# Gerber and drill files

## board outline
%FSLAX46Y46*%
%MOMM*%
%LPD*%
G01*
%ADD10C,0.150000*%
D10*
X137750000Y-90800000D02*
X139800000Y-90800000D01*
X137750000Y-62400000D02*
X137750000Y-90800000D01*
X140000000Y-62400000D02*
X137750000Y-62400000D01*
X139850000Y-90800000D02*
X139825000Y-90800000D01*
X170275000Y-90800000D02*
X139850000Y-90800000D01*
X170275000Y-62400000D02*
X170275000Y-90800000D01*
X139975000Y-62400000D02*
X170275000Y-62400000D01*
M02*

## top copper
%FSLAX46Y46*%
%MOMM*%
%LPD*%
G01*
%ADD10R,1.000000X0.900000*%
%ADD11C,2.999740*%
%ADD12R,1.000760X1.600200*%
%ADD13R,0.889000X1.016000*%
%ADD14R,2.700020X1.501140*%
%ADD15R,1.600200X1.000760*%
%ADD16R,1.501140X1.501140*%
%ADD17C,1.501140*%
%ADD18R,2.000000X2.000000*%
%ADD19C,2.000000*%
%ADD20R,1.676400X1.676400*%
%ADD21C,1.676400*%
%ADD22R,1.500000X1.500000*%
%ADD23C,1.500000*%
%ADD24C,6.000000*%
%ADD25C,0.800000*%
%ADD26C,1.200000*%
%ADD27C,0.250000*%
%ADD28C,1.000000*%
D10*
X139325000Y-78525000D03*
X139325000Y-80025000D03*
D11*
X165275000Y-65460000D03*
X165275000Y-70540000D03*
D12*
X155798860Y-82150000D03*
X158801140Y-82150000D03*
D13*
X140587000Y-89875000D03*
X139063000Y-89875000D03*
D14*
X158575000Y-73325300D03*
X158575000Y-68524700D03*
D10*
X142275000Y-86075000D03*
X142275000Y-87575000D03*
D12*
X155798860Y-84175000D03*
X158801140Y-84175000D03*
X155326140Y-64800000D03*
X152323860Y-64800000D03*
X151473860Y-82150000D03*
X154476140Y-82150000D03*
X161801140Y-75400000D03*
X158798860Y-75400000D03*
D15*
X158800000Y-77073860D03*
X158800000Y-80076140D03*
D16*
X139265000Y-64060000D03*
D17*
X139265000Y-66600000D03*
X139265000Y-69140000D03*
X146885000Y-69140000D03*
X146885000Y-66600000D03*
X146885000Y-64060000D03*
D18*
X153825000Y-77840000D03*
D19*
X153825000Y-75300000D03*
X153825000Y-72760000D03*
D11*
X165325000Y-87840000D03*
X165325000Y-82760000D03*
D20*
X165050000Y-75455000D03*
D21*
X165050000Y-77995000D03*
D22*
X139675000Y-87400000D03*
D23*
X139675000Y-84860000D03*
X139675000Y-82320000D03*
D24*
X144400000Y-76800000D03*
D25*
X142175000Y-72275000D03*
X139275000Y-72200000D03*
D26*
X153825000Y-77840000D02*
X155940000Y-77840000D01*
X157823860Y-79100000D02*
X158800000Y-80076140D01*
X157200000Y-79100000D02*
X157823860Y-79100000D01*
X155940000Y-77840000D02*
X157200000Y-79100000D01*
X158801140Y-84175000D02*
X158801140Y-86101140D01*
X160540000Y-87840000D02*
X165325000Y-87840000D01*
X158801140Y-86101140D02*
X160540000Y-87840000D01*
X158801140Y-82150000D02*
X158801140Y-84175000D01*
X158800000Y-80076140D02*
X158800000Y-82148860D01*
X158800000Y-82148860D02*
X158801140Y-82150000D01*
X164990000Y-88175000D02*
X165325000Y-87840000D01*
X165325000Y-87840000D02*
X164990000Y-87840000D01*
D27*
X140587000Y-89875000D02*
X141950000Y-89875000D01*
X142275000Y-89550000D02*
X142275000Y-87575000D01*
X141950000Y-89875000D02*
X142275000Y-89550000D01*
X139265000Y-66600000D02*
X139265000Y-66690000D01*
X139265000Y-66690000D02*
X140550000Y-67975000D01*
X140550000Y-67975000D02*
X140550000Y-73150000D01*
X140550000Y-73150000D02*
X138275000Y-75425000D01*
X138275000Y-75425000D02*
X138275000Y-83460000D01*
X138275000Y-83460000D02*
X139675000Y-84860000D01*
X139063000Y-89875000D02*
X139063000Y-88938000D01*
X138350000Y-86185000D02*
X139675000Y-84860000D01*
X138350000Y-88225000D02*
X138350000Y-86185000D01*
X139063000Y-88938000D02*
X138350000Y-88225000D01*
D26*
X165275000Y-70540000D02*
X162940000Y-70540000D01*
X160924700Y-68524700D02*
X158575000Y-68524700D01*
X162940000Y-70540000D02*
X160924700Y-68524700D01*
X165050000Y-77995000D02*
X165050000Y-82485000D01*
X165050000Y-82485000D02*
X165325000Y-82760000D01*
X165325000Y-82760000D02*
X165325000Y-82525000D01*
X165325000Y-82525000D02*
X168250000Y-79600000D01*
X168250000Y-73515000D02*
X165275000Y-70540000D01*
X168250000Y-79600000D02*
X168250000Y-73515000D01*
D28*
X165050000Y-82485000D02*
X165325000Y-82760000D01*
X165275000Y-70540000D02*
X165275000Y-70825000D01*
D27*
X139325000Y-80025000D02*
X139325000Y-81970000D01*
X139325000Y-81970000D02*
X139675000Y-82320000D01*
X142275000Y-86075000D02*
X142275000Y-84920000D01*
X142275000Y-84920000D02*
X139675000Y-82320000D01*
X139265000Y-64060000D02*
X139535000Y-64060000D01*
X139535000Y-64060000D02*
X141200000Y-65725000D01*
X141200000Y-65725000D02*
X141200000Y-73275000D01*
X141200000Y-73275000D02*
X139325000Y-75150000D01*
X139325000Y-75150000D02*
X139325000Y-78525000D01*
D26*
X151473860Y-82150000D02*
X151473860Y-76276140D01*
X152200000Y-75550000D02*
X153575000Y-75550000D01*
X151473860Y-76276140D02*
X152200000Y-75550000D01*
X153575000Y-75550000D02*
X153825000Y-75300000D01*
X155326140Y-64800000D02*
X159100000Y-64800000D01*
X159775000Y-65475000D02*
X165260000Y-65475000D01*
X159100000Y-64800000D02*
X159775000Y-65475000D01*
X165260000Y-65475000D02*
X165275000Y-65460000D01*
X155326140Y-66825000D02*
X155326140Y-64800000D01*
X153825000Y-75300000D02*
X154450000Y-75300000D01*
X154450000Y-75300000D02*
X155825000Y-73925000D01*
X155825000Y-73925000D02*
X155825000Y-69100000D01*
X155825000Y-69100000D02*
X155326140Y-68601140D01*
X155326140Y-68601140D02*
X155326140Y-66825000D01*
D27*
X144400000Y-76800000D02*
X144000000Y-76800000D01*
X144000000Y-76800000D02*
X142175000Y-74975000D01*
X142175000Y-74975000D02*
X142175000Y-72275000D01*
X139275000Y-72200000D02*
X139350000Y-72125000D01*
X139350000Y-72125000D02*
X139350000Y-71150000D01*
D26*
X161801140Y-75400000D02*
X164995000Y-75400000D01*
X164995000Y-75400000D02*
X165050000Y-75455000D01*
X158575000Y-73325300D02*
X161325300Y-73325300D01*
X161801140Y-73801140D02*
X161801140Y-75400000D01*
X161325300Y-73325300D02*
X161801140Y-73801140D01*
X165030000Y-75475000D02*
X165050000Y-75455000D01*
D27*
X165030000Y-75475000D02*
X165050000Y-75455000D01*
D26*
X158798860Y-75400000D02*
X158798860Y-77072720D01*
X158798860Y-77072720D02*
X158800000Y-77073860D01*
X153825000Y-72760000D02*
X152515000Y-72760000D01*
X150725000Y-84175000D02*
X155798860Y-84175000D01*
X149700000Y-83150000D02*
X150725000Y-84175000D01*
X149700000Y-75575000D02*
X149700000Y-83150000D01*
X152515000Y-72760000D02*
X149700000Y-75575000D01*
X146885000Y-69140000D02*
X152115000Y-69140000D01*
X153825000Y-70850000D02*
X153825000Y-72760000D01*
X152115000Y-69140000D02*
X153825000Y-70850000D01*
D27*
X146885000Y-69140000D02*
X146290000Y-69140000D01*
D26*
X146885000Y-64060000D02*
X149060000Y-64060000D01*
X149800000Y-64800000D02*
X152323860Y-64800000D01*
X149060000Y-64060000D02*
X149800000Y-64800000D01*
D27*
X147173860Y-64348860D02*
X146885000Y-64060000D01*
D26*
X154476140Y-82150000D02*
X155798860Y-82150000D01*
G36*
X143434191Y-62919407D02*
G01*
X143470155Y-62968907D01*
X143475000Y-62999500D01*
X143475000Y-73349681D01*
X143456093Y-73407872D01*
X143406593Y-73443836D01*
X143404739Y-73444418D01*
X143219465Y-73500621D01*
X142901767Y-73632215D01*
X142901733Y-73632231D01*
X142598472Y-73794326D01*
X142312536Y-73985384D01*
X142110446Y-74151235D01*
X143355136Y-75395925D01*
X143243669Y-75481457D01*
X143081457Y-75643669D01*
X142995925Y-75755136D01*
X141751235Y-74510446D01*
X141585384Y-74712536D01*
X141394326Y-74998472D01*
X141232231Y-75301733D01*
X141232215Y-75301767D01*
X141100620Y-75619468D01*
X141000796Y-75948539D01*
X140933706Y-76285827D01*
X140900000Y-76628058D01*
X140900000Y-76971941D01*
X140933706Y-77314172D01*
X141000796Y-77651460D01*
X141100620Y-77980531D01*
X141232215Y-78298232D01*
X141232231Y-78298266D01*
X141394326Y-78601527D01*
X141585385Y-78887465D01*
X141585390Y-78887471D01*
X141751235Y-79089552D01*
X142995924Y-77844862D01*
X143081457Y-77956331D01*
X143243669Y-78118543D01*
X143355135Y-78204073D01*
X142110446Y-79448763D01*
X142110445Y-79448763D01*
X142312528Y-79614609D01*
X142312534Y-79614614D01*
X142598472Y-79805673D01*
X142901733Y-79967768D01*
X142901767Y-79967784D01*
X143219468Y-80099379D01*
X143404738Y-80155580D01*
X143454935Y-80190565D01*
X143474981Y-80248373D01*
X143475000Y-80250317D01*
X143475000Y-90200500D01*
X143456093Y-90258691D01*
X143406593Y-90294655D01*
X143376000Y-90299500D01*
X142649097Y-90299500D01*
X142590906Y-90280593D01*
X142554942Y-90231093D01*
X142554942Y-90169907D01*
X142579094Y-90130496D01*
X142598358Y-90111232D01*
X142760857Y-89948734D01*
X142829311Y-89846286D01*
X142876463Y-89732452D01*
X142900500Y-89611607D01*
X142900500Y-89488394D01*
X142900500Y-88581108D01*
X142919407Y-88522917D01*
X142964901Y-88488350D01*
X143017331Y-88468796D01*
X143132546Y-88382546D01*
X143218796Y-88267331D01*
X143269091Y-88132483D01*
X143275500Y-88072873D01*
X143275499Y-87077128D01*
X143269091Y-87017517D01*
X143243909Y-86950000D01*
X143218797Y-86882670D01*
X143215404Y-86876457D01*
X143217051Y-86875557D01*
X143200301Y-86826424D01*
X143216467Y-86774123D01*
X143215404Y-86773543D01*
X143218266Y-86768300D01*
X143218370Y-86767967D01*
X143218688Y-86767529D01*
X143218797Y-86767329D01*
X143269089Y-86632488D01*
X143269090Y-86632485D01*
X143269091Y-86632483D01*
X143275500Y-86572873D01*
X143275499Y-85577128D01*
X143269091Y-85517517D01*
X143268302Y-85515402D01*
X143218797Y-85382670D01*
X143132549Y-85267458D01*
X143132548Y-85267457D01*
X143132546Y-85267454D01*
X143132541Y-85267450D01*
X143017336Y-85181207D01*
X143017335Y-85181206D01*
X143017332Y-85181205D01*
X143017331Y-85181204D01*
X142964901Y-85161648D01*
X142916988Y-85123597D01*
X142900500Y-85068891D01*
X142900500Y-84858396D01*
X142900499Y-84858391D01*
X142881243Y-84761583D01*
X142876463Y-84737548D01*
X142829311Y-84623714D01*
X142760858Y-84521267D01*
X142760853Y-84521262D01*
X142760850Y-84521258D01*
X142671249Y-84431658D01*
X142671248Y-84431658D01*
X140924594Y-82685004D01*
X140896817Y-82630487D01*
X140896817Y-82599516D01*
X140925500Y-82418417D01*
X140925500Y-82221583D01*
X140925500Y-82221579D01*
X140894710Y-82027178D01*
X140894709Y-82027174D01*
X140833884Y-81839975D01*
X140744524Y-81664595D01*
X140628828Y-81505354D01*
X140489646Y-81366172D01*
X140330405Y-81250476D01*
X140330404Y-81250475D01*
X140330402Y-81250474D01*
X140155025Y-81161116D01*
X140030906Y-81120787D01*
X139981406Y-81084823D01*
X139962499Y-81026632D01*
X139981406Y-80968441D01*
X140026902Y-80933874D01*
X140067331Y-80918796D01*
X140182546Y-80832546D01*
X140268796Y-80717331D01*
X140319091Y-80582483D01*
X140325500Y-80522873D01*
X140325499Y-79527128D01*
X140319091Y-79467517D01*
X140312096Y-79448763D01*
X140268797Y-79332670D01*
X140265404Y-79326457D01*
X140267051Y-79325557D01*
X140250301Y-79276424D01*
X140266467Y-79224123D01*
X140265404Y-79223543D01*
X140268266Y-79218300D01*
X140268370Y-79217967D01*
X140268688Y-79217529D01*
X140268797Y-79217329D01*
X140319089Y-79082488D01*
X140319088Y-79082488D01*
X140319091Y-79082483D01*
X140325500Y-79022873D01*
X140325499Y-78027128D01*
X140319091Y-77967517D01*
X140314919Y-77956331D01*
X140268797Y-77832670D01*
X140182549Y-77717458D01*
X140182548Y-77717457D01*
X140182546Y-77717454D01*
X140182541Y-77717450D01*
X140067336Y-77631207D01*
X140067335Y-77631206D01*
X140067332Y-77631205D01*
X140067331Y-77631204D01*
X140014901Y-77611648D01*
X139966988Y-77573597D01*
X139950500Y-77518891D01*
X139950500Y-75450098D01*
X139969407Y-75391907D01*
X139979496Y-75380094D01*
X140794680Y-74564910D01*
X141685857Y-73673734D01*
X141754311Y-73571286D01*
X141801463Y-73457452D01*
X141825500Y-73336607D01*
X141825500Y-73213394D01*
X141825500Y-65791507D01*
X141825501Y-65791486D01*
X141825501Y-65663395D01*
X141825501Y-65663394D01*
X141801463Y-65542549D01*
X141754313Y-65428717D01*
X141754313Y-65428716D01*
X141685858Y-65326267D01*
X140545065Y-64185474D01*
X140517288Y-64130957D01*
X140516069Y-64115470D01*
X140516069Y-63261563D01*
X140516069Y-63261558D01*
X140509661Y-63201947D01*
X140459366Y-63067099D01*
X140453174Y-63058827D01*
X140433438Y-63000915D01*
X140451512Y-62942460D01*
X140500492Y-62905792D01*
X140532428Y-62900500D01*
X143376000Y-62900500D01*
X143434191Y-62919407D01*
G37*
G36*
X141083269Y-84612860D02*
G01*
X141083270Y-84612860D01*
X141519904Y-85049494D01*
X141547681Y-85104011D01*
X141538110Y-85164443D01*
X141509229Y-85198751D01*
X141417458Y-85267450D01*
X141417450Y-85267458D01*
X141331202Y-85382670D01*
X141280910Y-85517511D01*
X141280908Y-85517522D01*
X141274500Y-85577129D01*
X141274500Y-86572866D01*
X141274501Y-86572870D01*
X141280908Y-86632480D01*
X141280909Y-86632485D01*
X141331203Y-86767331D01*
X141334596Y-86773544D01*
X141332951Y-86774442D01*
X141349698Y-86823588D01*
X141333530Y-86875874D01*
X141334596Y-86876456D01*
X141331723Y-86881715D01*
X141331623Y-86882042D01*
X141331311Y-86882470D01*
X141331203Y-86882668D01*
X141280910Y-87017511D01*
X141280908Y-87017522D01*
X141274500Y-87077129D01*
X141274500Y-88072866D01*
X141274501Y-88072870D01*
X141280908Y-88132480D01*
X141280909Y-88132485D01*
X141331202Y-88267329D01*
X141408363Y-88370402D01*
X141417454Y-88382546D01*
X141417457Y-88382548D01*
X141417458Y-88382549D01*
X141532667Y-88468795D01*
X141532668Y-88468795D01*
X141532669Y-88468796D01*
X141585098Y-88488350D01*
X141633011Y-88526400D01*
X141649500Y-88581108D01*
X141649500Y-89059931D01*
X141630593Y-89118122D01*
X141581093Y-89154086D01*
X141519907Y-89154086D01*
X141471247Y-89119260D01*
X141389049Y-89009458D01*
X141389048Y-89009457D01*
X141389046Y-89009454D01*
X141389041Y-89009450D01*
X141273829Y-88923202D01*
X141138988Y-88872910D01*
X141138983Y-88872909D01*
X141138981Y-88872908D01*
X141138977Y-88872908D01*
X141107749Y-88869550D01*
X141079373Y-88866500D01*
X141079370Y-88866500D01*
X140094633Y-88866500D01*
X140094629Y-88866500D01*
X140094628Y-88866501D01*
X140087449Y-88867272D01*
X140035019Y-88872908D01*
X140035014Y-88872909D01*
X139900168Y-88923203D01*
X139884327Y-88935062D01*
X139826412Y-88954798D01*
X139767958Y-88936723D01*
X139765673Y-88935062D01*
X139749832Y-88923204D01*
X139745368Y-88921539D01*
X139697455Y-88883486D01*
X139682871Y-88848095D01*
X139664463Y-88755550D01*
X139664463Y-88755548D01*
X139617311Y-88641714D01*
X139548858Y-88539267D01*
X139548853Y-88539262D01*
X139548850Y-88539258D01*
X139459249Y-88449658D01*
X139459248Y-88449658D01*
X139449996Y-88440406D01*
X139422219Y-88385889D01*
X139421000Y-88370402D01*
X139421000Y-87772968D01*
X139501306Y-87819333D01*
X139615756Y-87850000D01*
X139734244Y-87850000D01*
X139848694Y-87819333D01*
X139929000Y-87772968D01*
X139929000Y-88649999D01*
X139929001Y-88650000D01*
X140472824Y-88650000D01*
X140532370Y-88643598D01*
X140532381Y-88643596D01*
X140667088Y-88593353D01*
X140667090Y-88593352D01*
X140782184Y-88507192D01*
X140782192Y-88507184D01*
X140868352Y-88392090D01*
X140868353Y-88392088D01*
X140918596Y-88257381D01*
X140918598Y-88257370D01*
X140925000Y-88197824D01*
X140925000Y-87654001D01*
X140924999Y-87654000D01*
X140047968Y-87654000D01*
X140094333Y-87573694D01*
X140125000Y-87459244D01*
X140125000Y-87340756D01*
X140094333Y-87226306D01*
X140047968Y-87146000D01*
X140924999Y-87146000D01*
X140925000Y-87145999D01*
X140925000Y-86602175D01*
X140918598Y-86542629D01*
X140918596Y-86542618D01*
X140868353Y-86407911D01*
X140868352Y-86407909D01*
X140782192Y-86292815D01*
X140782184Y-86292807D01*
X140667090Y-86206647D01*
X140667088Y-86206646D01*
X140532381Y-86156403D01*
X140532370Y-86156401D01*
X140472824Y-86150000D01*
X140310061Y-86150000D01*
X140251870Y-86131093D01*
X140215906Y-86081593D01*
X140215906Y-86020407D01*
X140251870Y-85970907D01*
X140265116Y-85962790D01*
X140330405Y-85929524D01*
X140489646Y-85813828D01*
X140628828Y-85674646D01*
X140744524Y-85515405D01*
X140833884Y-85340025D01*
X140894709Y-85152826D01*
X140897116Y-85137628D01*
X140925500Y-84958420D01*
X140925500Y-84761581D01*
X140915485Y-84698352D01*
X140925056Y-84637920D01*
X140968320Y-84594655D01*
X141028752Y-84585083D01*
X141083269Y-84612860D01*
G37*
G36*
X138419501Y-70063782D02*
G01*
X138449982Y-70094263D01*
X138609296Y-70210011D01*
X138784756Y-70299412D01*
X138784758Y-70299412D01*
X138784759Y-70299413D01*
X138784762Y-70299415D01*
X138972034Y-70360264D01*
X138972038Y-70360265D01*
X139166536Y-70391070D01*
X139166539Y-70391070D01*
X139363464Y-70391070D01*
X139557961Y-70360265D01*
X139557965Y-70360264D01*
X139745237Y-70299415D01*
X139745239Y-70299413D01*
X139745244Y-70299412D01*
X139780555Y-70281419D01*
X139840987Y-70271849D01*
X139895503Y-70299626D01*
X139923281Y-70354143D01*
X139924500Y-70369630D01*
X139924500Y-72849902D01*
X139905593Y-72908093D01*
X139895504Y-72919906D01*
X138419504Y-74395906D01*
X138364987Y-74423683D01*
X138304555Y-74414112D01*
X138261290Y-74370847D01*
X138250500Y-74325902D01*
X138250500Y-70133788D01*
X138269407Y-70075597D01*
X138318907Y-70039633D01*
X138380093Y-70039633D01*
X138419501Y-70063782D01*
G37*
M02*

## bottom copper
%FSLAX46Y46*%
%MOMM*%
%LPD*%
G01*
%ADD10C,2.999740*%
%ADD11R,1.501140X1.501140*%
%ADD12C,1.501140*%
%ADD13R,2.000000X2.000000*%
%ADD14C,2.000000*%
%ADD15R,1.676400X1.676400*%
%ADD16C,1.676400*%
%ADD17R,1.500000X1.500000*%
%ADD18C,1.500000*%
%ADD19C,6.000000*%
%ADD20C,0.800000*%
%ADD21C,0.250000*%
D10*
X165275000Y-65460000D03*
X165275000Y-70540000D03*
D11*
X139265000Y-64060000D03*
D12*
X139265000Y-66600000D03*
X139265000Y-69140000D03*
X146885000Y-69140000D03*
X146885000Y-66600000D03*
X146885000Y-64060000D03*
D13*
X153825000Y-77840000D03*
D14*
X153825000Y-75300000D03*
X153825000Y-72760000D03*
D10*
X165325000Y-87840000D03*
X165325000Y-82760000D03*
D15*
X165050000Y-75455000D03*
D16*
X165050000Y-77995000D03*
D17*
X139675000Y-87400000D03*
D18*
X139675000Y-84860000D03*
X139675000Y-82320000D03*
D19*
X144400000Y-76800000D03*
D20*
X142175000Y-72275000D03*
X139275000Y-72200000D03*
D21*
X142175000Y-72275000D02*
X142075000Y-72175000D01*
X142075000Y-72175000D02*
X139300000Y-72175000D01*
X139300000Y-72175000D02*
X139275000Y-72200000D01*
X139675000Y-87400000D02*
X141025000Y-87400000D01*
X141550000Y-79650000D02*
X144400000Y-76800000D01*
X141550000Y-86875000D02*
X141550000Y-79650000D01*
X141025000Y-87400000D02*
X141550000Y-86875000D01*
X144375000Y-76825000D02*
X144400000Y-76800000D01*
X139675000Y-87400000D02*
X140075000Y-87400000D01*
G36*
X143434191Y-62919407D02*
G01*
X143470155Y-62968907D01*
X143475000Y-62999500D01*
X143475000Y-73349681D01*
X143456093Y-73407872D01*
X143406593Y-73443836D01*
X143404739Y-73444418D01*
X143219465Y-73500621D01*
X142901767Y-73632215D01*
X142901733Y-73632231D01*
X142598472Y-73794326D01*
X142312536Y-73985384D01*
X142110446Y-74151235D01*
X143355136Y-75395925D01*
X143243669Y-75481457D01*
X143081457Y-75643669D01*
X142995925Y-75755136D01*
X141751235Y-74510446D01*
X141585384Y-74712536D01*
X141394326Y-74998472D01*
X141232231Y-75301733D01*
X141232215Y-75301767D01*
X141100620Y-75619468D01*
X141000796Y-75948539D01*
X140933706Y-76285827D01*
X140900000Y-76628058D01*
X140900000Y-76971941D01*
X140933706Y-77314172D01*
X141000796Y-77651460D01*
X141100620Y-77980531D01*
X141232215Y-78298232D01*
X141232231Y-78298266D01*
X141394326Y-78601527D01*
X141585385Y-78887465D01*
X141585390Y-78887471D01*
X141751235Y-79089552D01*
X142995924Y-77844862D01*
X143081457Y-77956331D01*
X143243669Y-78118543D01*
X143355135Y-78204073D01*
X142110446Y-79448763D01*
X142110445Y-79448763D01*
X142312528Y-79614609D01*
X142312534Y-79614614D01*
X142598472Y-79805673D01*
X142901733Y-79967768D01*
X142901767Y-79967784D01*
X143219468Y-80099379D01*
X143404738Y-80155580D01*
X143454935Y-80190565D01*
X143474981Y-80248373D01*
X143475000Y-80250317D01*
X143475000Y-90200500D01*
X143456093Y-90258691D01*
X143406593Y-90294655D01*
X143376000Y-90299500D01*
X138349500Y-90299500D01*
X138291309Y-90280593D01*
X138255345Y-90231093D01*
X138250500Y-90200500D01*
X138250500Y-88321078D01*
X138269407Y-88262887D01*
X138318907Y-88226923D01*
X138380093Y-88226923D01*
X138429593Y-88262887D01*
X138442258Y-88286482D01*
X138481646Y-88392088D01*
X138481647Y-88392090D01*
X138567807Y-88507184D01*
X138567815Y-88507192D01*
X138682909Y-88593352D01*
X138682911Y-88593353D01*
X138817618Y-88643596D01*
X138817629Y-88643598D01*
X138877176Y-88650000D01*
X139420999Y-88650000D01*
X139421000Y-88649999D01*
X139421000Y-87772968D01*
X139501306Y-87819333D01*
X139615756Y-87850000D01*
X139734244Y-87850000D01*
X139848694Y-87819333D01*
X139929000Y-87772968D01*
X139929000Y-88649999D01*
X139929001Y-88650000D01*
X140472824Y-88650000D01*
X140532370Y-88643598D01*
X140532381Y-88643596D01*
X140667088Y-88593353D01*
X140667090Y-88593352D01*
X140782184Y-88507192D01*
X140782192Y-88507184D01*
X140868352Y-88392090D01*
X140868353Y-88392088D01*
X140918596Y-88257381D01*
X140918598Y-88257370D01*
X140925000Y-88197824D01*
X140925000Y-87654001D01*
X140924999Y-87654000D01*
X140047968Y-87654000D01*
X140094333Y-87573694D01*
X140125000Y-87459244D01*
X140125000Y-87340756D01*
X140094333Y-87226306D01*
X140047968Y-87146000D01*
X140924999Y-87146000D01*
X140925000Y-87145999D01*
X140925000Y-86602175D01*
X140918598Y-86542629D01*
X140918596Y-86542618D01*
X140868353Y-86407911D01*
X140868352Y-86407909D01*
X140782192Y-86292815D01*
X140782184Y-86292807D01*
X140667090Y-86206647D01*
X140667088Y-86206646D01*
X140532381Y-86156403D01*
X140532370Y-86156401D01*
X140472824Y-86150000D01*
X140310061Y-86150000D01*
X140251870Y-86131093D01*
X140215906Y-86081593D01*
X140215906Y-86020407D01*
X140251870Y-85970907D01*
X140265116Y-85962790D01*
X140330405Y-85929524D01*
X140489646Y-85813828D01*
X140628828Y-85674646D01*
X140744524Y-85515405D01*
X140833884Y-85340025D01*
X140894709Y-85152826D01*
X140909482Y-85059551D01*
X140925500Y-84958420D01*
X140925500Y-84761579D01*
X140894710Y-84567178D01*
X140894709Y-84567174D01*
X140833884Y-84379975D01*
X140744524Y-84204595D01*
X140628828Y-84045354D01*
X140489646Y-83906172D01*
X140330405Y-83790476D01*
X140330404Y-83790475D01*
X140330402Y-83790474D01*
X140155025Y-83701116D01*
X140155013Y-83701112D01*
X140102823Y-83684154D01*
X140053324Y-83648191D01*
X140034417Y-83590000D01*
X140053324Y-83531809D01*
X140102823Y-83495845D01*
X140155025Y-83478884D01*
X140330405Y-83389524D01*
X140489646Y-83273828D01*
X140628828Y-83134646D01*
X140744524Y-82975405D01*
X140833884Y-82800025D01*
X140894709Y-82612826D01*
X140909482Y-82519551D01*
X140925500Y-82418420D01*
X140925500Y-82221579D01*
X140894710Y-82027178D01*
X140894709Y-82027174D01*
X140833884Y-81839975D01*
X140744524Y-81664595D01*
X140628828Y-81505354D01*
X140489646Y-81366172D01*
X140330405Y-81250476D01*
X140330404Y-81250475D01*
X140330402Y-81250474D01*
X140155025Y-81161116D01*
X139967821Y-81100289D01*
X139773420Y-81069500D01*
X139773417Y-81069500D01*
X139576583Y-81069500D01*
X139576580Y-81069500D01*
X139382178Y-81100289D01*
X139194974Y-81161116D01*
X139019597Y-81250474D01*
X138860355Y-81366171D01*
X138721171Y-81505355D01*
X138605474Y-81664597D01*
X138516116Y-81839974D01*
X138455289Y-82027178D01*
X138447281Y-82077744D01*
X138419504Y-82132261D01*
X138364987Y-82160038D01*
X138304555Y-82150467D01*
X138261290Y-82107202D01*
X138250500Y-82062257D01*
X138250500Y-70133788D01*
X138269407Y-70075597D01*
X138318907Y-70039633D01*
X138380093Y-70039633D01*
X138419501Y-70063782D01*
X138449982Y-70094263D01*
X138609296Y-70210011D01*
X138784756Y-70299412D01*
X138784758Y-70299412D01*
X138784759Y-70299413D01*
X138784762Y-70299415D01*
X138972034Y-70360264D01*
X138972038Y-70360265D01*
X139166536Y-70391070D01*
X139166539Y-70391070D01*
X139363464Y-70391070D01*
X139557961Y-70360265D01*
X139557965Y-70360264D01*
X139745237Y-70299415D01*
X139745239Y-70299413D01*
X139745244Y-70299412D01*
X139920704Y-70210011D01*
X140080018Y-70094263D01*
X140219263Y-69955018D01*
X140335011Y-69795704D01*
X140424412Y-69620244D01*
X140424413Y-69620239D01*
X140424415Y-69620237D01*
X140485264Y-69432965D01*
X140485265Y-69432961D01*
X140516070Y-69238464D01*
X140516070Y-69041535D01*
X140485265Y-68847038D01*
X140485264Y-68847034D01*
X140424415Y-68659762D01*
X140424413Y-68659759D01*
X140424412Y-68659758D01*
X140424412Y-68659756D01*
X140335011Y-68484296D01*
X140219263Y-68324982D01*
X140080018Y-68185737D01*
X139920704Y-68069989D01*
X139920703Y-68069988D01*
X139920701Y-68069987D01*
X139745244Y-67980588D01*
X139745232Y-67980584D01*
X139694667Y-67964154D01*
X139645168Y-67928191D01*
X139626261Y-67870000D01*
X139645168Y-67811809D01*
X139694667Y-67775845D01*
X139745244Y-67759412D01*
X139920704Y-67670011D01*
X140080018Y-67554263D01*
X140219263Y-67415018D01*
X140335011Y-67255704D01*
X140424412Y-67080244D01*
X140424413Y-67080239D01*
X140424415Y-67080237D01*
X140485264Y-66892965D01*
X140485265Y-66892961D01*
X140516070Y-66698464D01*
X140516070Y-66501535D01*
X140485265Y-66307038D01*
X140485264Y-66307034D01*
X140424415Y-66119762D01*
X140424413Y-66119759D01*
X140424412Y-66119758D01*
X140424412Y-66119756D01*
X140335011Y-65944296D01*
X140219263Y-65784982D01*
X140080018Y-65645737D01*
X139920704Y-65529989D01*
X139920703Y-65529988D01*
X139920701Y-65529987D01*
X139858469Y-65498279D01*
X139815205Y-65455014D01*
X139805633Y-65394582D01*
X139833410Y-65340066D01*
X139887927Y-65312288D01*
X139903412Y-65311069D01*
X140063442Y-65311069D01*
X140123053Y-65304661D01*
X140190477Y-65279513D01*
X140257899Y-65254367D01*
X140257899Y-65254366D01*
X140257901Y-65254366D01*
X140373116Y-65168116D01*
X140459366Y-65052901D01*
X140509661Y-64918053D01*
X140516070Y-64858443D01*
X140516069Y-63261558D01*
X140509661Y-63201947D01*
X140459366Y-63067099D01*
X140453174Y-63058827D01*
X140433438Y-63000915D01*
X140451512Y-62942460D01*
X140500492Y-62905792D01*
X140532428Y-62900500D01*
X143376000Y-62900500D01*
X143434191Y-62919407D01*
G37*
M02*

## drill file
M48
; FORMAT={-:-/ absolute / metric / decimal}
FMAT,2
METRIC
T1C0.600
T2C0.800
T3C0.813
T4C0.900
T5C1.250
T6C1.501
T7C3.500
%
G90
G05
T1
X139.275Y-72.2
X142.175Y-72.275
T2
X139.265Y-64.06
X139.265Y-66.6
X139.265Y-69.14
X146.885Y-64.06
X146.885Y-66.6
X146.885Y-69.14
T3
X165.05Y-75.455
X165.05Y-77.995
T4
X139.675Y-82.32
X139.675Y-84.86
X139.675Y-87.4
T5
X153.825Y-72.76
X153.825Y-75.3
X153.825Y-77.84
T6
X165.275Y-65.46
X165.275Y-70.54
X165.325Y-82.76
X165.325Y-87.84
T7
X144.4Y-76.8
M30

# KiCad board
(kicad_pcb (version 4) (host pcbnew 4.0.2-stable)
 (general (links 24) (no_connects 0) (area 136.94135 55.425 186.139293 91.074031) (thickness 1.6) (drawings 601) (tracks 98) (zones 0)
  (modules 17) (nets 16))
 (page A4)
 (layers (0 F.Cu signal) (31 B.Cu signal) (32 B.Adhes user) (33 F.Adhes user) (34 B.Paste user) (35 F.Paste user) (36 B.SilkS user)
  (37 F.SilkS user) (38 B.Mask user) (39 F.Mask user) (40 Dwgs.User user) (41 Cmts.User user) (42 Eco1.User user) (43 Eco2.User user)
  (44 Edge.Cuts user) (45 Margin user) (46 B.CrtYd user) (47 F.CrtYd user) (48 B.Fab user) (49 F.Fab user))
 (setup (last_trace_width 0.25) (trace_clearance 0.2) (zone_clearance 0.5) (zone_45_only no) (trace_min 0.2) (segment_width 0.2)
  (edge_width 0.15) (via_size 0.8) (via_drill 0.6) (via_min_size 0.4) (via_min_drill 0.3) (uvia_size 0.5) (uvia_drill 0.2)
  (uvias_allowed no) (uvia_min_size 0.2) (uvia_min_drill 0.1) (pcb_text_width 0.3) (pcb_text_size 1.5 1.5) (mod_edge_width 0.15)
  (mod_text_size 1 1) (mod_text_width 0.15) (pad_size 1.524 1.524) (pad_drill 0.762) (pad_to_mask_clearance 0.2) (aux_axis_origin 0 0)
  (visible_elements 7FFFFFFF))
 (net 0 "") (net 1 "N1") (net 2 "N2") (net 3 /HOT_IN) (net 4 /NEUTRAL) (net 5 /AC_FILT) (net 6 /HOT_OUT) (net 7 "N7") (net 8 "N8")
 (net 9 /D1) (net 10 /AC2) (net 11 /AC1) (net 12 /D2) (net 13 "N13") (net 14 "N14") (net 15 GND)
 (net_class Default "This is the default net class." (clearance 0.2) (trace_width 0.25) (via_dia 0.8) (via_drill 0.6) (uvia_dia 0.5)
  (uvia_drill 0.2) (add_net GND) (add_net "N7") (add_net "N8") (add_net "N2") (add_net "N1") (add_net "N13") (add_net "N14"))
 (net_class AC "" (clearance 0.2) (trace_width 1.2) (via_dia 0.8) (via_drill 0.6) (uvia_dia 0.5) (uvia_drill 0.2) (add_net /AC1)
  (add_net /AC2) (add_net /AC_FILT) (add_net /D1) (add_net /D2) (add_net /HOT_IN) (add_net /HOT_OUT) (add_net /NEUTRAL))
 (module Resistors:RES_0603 (layer F.Cu) (at 139.325 79.275 270)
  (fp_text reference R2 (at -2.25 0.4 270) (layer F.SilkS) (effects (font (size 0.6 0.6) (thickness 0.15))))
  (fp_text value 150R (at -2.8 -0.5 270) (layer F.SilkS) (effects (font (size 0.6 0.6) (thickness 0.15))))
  (pad 1 smd rect (at -0.75 0 270) (size 0.9 1) (layers F.Cu F.Paste F.Mask) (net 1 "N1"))
  (pad 2 smd rect (at 0.75 0 270) (size 0.9 1) (layers F.Cu F.Paste F.Mask) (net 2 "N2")))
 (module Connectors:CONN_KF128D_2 (layer F.Cu) (at 165.275 68 270)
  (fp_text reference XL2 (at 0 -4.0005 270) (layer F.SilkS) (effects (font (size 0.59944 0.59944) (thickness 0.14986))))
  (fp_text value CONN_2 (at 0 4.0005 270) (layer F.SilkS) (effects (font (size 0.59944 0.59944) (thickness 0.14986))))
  (pad 1 thru_hole circle (at -2.54 0 270) (size 2.99974 2.99974) (drill 1.50114) (layers *.Cu *.Mask F.SilkS) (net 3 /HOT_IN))
  (pad 2 thru_hole circle (at 2.54 0 270) (size 2.99974 2.99974) (drill 1.50114) (layers *.Cu *.Mask F.SilkS) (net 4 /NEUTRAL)))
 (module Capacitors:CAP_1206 (layer F.Cu) (at 157.3 82.15)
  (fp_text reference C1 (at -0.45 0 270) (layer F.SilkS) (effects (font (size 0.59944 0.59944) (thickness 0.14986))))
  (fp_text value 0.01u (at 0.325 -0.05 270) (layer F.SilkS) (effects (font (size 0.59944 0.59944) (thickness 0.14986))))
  (pad 1 smd rect (at -1.50114 0) (size 1.00076 1.6002) (layers F.Cu F.Paste F.Mask) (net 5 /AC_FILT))
  (pad 2 smd rect (at 1.50114 0) (size 1.00076 1.6002) (layers F.Cu F.Paste F.Mask) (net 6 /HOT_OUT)))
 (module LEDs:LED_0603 (layer F.Cu) (at 139.825 89.875 180)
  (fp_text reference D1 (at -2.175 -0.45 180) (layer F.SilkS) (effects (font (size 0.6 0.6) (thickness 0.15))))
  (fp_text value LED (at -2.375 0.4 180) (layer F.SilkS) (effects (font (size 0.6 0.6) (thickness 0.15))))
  (pad A smd rect (at -0.762 0 180) (size 0.889 1.016) (layers F.Cu F.Paste F.Mask) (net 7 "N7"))
  (pad C smd rect (at 0.762 0 180) (size 0.889 1.016) (layers F.Cu F.Paste F.Mask) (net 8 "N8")))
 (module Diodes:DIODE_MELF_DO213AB (layer F.Cu) (at 158.575 70.925 90)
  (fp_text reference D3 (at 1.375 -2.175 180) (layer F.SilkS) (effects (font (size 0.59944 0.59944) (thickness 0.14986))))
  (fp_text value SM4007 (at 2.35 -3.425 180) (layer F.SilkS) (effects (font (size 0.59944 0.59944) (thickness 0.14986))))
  (pad C smd rect (at -2.4003 0 90) (size 1.50114 2.70002) (layers F.Cu F.Paste F.Mask) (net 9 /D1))
  (pad A smd rect (at 2.4003 0 90) (size 1.50114 2.70002) (layers F.Cu F.Paste F.Mask) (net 4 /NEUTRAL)))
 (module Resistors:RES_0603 (layer F.Cu) (at 142.275 86.825 270)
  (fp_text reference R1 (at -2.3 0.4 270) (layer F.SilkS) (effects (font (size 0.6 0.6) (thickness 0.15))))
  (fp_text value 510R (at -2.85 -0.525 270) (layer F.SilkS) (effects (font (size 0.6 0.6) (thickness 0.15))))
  (pad 1 smd rect (at -0.75 0 270) (size 0.9 1) (layers F.Cu F.Paste F.Mask) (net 2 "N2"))
  (pad 2 smd rect (at 0.75 0 270) (size 0.9 1) (layers F.Cu F.Paste F.Mask) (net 7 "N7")))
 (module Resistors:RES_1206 (layer F.Cu) (at 157.3 84.175)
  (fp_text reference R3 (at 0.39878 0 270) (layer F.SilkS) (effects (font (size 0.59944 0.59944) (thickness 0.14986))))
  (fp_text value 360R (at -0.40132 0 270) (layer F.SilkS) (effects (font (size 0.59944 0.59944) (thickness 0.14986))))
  (pad 1 smd rect (at -1.50114 0) (size 1.00076 1.6002) (layers F.Cu F.Paste F.Mask) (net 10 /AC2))
  (pad 2 smd rect (at 1.50114 0) (size 1.00076 1.6002) (layers F.Cu F.Paste F.Mask) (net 6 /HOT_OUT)))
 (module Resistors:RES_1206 (layer F.Cu) (at 153.825 64.8 180)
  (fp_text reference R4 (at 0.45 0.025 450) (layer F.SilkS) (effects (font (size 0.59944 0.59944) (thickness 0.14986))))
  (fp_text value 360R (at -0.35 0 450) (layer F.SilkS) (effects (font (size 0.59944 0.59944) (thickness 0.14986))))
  (pad 1 smd rect (at -1.50114 0 180) (size 1.00076 1.6002) (layers F.Cu F.Paste F.Mask) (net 3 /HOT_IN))
  (pad 2 smd rect (at 1.50114 0 180) (size 1.00076 1.6002) (layers F.Cu F.Paste F.Mask) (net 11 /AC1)))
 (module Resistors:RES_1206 (layer F.Cu) (at 152.975 82.15)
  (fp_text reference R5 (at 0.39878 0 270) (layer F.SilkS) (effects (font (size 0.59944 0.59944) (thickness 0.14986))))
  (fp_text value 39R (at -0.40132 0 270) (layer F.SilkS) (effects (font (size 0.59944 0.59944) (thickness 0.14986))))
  (pad 1 smd rect (at -1.50114 0) (size 1.00076 1.6002) (layers F.Cu F.Paste F.Mask) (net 3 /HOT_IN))
  (pad 2 smd rect (at 1.50114 0) (size 1.00076 1.6002) (layers F.Cu F.Paste F.Mask) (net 5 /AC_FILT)))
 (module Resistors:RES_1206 (layer F.Cu) (at 160.3 75.4 180)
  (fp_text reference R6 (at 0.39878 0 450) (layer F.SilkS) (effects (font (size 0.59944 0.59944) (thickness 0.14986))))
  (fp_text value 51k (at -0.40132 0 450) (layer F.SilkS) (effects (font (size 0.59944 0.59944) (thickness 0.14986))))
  (pad 1 smd rect (at -1.50114 0 180) (size 1.00076 1.6002) (layers F.Cu F.Paste F.Mask) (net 9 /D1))
  (pad 2 smd rect (at 1.50114 0 180) (size 1.00076 1.6002) (layers F.Cu F.Paste F.Mask) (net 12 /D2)))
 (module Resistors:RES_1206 (layer F.Cu) (at 158.8 78.575 270)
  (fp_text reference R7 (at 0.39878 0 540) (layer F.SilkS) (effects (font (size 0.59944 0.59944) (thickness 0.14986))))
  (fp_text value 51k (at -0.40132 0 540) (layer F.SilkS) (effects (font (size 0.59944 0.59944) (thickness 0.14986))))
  (pad 1 smd rect (at -1.50114 0 270) (size 1.00076 1.6002) (layers F.Cu F.Paste F.Mask) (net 12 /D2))
  (pad 2 smd rect (at 1.50114 0 270) (size 1.00076 1.6002) (layers F.Cu F.Paste F.Mask) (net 6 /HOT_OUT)))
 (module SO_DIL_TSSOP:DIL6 (layer F.Cu) (at 143.075 66.6 270)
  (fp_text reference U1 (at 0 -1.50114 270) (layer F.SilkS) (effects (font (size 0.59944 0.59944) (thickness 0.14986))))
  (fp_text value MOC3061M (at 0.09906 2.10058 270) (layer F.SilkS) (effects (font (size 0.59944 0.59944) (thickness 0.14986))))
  (pad 1 thru_hole rect (at -2.54 3.81 270) (size 1.50114 1.50114) (drill 0.8001) (layers *.Cu *.Mask F.SilkS) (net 1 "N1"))
  (pad 2 thru_hole circle (at 0 3.81 270) (size 1.50114 1.50114) (drill 0.8001) (layers *.Cu *.Mask F.SilkS) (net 8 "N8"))
  (pad 3 thru_hole circle (at 2.54 3.81 270) (size 1.50114 1.50114) (drill 0.8001) (layers *.Cu *.Mask F.SilkS) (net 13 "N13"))
  (pad 4 thru_hole circle (at 2.54 -3.81 270) (size 1.50114 1.50114) (drill 0.8001) (layers *.Cu *.Mask F.SilkS) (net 10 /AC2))
  (pad 5 thru_hole circle (at 0 -3.81 270) (size 1.50114 1.50114) (drill 0.8001) (layers *.Cu *.Mask F.SilkS) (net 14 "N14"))
  (pad 6 thru_hole circle (at -2.54 -3.81 270) (size 1.50114 1.50114) (drill 0.8001) (layers *.Cu *.Mask F.SilkS) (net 11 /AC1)))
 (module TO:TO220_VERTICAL (layer F.Cu) (at 153.825 75.3 90)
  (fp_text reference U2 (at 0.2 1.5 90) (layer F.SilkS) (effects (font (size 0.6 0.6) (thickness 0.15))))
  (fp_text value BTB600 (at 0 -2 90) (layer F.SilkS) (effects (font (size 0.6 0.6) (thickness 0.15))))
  (pad 1 thru_hole rect (at -2.54 0 90) (size 2 2) (drill 1.25) (layers *.Cu *.Mask F.SilkS) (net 6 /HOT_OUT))
  (pad 2 thru_hole circle (at 0 0 90) (size 2 2) (drill 1.25) (layers *.Cu *.Mask F.SilkS) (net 3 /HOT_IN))
  (pad 3 thru_hole circle (at 2.54 0 90) (size 2 2) (drill 1.25) (layers *.Cu *.Mask F.SilkS) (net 10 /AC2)))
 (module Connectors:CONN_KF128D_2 (layer F.Cu) (at 165.325 85.3 90)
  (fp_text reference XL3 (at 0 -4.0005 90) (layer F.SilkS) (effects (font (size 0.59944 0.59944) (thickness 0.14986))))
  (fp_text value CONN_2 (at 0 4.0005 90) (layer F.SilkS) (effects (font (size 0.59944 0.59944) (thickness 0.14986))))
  (pad 1 thru_hole circle (at -2.54 0 90) (size 2.99974 2.99974) (drill 1.50114) (layers *.Cu *.Mask F.SilkS) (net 6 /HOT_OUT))
  (pad 2 thru_hole circle (at 2.54 0 90) (size 2.99974 2.99974) (drill 1.50114) (layers *.Cu *.Mask F.SilkS) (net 4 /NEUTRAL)))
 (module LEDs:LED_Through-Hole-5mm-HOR (layer F.Cu) (at 165.05 76.725 270)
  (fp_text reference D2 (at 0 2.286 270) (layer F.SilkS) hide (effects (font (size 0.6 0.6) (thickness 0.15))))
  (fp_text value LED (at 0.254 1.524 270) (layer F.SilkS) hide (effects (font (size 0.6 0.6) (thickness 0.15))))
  (pad A thru_hole rect (at -1.27 0 270) (size 1.6764 1.6764) (drill 0.8128) (layers *.Cu *.Mask F.SilkS) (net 9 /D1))
  (pad C thru_hole circle (at 1.27 0 270) (size 1.6764 1.6764) (drill 0.8128) (layers *.Cu *.Mask F.SilkS) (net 4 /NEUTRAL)))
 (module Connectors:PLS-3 (layer F.Cu) (at 139.675 87.4 90)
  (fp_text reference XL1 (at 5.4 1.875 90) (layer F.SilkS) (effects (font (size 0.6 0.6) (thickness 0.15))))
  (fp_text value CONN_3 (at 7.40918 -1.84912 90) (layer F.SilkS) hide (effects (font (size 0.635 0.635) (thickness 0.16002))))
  (pad 1 thru_hole rect (at 0 0 90) (size 1.5 1.5) (drill 0.9) (layers *.Cu *.Mask F.SilkS) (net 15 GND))
  (pad 2 thru_hole circle (at 2.54 0 90) (size 1.5 1.5) (drill 0.9) (layers *.Cu *.Mask F.SilkS) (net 8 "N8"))
  (pad 3 thru_hole circle (at 5.08 0 90) (size 1.5 1.5) (drill 0.9) (layers *.Cu *.Mask F.SilkS) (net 2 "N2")))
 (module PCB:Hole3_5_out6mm (layer F.Cu) (at 144.4 76.8)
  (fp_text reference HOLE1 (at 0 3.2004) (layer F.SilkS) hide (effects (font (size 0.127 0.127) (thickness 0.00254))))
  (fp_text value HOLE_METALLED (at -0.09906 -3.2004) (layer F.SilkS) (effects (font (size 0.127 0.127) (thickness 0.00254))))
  (pad H thru_hole circle (at 0 0) (size 6 6) (drill 3.5) (layers *.Cu *.Mask F.SilkS) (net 15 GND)))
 (gr_line (start 137.75 90.8) (end 139.8 90.8) (angle 90) (layer Edge.Cuts) (width 0.15))
 (gr_line (start 137.75 62.4) (end 137.75 90.8) (angle 90) (layer Edge.Cuts) (width 0.15))
 (gr_line (start 140 62.4) (end 137.75 62.4) (angle 90) (layer Edge.Cuts) (width 0.15))
 (gr_line (start 139.85 90.8) (end 139.825 90.8) (angle 90) (layer Edge.Cuts) (width 0.15))
 (gr_line (start 170.275 90.8) (end 139.85 90.8) (angle 90) (layer Edge.Cuts) (width 0.15))
 (gr_line (start 170.275 62.4) (end 170.275 90.8) (angle 90) (layer Edge.Cuts) (width 0.15))
 (gr_line (start 139.975 62.4) (end 170.275 62.4) (angle 90) (layer Edge.Cuts) (width 0.15))
 (segment (start 153.825 77.84) (end 155.94 77.84) (width 1.2) (layer F.Cu) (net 6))
 (segment (start 157.82386 79.1) (end 158.8 80.07614) (width 1.2) (layer F.Cu) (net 6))
 (segment (start 157.2 79.1) (end 157.82386 79.1) (width 1.2) (layer F.Cu) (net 6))
 (segment (start 155.94 77.84) (end 157.2 79.1) (width 1.2) (layer F.Cu) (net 6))
 (segment (start 158.80114 84.175) (end 158.80114 86.10114) (width 1.2) (layer F.Cu) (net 6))
 (segment (start 160.54 87.84) (end 165.325 87.84) (width 1.2) (layer F.Cu) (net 6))
 (segment (start 158.80114 86.10114) (end 160.54 87.84) (width 1.2) (layer F.Cu) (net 6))
 (segment (start 158.80114 82.15) (end 158.80114 84.175) (width 1.2) (layer F.Cu) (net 6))
 (segment (start 158.8 80.07614) (end 158.8 82.14886) (width 1.2) (layer F.Cu) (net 6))
 (segment (start 158.8 82.14886) (end 158.80114 82.15) (width 1.2) (layer F.Cu) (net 6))
 (segment (start 164.99 88.175) (end 165.325 87.84) (width 1.2) (layer F.Cu) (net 6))
 (segment (start 165.325 87.84) (end 164.99 87.84) (width 1.2) (layer F.Cu) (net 6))
 (segment (start 140.587 89.875) (end 141.95 89.875) (width 0.25) (layer F.Cu) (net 7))
 (segment (start 142.275 89.55) (end 142.275 87.575) (width 0.25) (layer F.Cu) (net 7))
 (segment (start 141.95 89.875) (end 142.275 89.55) (width 0.25) (layer F.Cu) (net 7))
 (segment (start 139.265 66.6) (end 139.265 66.69) (width 0.25) (layer F.Cu) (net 8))
 (segment (start 139.265 66.69) (end 140.55 67.975) (width 0.25) (layer F.Cu) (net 8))
 (segment (start 140.55 67.975) (end 140.55 73.15) (width 0.25) (layer F.Cu) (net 8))
 (segment (start 140.55 73.15) (end 138.275 75.425) (width 0.25) (layer F.Cu) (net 8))
 (segment (start 138.275 75.425) (end 138.275 83.46) (width 0.25) (layer F.Cu) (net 8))
 (segment (start 138.275 83.46) (end 139.675 84.86) (width 0.25) (layer F.Cu) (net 8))
 (segment (start 139.063 89.875) (end 139.063 88.938) (width 0.25) (layer F.Cu) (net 8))
 (segment (start 138.35 86.185) (end 139.675 84.86) (width 0.25) (layer F.Cu) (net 8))
 (segment (start 138.35 88.225) (end 138.35 86.185) (width 0.25) (layer F.Cu) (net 8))
 (segment (start 139.063 88.938) (end 138.35 88.225) (width 0.25) (layer F.Cu) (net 8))
 (segment (start 165.275 70.54) (end 162.94 70.54) (width 1.2) (layer F.Cu) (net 4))
 (segment (start 160.9247 68.5247) (end 158.575 68.5247) (width 1.2) (layer F.Cu) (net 4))
 (segment (start 162.94 70.54) (end 160.9247 68.5247) (width 1.2) (layer F.Cu) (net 4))
 (segment (start 165.05 77.995) (end 165.05 82.485) (width 1.2) (layer F.Cu) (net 4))
 (segment (start 165.05 82.485) (end 165.325 82.76) (width 1.2) (layer F.Cu) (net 4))
 (segment (start 165.325 82.76) (end 165.325 82.525) (width 1.2) (layer F.Cu) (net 4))
 (segment (start 165.325 82.525) (end 168.25 79.6) (width 1.2) (layer F.Cu) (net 4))
 (segment (start 168.25 73.515) (end 165.275 70.54) (width 1.2) (layer F.Cu) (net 4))
 (segment (start 168.25 79.6) (end 168.25 73.515) (width 1.2) (layer F.Cu) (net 4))
 (segment (start 165.05 82.485) (end 165.325 82.76) (width 1) (layer F.Cu) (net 4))
 (segment (start 165.275 70.54) (end 165.275 70.825) (width 1) (layer F.Cu) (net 4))
 (segment (start 139.325 80.025) (end 139.325 81.97) (width 0.25) (layer F.Cu) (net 2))
 (segment (start 139.325 81.97) (end 139.675 82.32) (width 0.25) (layer F.Cu) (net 2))
 (segment (start 142.275 86.075) (end 142.275 84.92) (width 0.25) (layer F.Cu) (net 2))
 (segment (start 142.275 84.92) (end 139.675 82.32) (width 0.25) (layer F.Cu) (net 2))
 (segment (start 139.265 64.06) (end 139.535 64.06) (width 0.25) (layer F.Cu) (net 1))
 (segment (start 139.535 64.06) (end 141.2 65.725) (width 0.25) (layer F.Cu) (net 1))
 (segment (start 141.2 65.725) (end 141.2 73.275) (width 0.25) (layer F.Cu) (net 1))
 (segment (start 141.2 73.275) (end 139.325 75.15) (width 0.25) (layer F.Cu) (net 1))
 (segment (start 139.325 75.15) (end 139.325 78.525) (width 0.25) (layer F.Cu) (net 1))
 (segment (start 151.47386 82.15) (end 151.47386 76.27614) (width 1.2) (layer F.Cu) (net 3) (status 400000))
 (segment (start 152.2 75.55) (end 153.575 75.55) (width 1.2) (layer F.Cu) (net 3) (status 800000))
 (segment (start 151.47386 76.27614) (end 152.2 75.55) (width 1.2) (layer F.Cu) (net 3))
 (segment (start 153.575 75.55) (end 153.825 75.3) (width 1.2) (layer F.Cu) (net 3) (status C00000))
 (segment (start 155.32614 64.8) (end 159.1 64.8) (width 1.2) (layer F.Cu) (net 3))
 (segment (start 159.775 65.475) (end 165.26 65.475) (width 1.2) (layer F.Cu) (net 3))
 (segment (start 159.1 64.8) (end 159.775 65.475) (width 1.2) (layer F.Cu) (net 3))
 (segment (start 165.26 65.475) (end 165.275 65.46) (width 1.2) (layer F.Cu) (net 3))
 (segment (start 155.32614 66.825) (end 155.32614 64.8) (width 1.2) (layer F.Cu) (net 3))
 (segment (start 153.825 75.3) (end 154.45 75.3) (width 1.2) (layer F.Cu) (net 3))
 (segment (start 154.45 75.3) (end 155.825 73.925) (width 1.2) (layer F.Cu) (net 3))
 (segment (start 155.825 73.925) (end 155.825 69.1) (width 1.2) (layer F.Cu) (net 3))
 (segment (start 155.825 69.1) (end 155.32614 68.60114) (width 1.2) (layer F.Cu) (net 3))
 (segment (start 155.32614 68.60114) (end 155.32614 66.825) (width 1.2) (layer F.Cu) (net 3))
 (segment (start 144.4 76.8) (end 144 76.8) (width 0.25) (layer F.Cu) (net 15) (status C00000))
 (segment (start 144 76.8) (end 142.175 74.975) (width 0.25) (layer F.Cu) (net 15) (status C00000))
 (segment (start 142.175 74.975) (end 142.175 72.275) (width 0.25) (layer F.Cu) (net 15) (status 400000))
 (via (at 142.175 72.275) (size 0.8) (drill 0.6) (layers F.Cu B.Cu) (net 15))
 (segment (start 142.175 72.275) (end 142.075 72.175) (width 0.25) (layer B.Cu) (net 15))
 (segment (start 142.075 72.175) (end 139.3 72.175) (width 0.25) (layer B.Cu) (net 15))
 (segment (start 139.3 72.175) (end 139.275 72.2) (width 0.25) (layer B.Cu) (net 15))
 (via (at 139.275 72.2) (size 0.8) (drill 0.6) (layers F.Cu B.Cu) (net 15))
 (segment (start 139.275 72.2) (end 139.35 72.125) (width 0.25) (layer F.Cu) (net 15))
 (segment (start 139.35 72.125) (end 139.35 71.15) (width 0.25) (layer F.Cu) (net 15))
 (segment (start 139.675 87.4) (end 141.025 87.4) (width 0.25) (layer B.Cu) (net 15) (status 400000))
 (segment (start 141.55 79.65) (end 144.4 76.8) (width 0.25) (layer B.Cu) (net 15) (status 800000))
 (segment (start 141.55 86.875) (end 141.55 79.65) (width 0.25) (layer B.Cu) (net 15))
 (segment (start 141.025 87.4) (end 141.55 86.875) (width 0.25) (layer B.Cu) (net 15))
 (segment (start 144.375 76.825) (end 144.4 76.8) (width 0.25) (layer B.Cu) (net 15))
 (segment (start 139.675 87.4) (end 140.075 87.4) (width 0.25) (layer B.Cu) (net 15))
 (segment (start 161.80114 75.4) (end 164.995 75.4) (width 1.2) (layer F.Cu) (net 9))
 (segment (start 164.995 75.4) (end 165.05 75.455) (width 1.2) (layer F.Cu) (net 9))
 (segment (start 158.575 73.3253) (end 161.3253 73.3253) (width 1.2) (layer F.Cu) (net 9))
 (segment (start 161.80114 73.80114) (end 161.80114 75.4) (width 1.2) (layer F.Cu) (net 9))
 (segment (start 161.3253 73.3253) (end 161.80114 73.80114) (width 1.2) (layer F.Cu) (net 9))
 (segment (start 165.03 75.475) (end 165.05 75.455) (width 1.2) (layer F.Cu) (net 9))
 (segment (start 165.03 75.475) (end 165.05 75.455) (width 0.25) (layer F.Cu) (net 9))
 (segment (start 158.79886 75.4) (end 158.79886 77.07272) (width 1.2) (layer F.Cu) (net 12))
 (segment (start 158.79886 77.07272) (end 158.8 77.07386) (width 1.2) (layer F.Cu) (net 12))
 (segment (start 153.825 72.76) (end 152.515 72.76) (width 1.2) (layer F.Cu) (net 10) (status 400000))
 (segment (start 150.725 84.175) (end 155.79886 84.175) (width 1.2) (layer F.Cu) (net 10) (status 800000))
 (segment (start 149.7 83.15) (end 150.725 84.175) (width 1.2) (layer F.Cu) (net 10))
 (segment (start 149.7 75.575) (end 149.7 83.15) (width 1.2) (layer F.Cu) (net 10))
 (segment (start 152.515 72.76) (end 149.7 75.575) (width 1.2) (layer F.Cu) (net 10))
 (segment (start 146.885 69.14) (end 152.115 69.14) (width 1.2) (layer F.Cu) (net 10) (status 400000))
 (segment (start 153.825 70.85) (end 153.825 72.76) (width 1.2) (layer F.Cu) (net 10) (status 800000))
 (segment (start 152.115 69.14) (end 153.825 70.85) (width 1.2) (layer F.Cu) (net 10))
 (segment (start 146.885 69.14) (end 146.29 69.14) (width 0.25) (layer F.Cu) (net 10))
 (segment (start 146.885 64.06) (end 149.06 64.06) (width 1.2) (layer F.Cu) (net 11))
 (segment (start 149.8 64.8) (end 152.32386 64.8) (width 1.2) (layer F.Cu) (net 11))
 (segment (start 149.06 64.06) (end 149.8 64.8) (width 1.2) (layer F.Cu) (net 11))
 (segment (start 147.17386 64.34886) (end 146.885 64.06) (width 0.25) (layer F.Cu) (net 11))
 (segment (start 154.47614 82.15) (end 155.79886 82.15) (width 1.2) (layer F.Cu) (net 5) (status C00000))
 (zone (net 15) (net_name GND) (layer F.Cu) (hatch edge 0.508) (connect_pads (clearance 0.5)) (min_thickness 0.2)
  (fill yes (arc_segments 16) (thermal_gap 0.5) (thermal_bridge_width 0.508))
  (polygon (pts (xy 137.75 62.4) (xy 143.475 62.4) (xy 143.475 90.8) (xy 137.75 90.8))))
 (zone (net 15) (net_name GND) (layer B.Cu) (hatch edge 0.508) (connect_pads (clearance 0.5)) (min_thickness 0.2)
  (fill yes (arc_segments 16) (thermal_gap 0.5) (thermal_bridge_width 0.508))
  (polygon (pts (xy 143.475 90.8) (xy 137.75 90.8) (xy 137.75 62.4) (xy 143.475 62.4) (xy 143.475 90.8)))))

